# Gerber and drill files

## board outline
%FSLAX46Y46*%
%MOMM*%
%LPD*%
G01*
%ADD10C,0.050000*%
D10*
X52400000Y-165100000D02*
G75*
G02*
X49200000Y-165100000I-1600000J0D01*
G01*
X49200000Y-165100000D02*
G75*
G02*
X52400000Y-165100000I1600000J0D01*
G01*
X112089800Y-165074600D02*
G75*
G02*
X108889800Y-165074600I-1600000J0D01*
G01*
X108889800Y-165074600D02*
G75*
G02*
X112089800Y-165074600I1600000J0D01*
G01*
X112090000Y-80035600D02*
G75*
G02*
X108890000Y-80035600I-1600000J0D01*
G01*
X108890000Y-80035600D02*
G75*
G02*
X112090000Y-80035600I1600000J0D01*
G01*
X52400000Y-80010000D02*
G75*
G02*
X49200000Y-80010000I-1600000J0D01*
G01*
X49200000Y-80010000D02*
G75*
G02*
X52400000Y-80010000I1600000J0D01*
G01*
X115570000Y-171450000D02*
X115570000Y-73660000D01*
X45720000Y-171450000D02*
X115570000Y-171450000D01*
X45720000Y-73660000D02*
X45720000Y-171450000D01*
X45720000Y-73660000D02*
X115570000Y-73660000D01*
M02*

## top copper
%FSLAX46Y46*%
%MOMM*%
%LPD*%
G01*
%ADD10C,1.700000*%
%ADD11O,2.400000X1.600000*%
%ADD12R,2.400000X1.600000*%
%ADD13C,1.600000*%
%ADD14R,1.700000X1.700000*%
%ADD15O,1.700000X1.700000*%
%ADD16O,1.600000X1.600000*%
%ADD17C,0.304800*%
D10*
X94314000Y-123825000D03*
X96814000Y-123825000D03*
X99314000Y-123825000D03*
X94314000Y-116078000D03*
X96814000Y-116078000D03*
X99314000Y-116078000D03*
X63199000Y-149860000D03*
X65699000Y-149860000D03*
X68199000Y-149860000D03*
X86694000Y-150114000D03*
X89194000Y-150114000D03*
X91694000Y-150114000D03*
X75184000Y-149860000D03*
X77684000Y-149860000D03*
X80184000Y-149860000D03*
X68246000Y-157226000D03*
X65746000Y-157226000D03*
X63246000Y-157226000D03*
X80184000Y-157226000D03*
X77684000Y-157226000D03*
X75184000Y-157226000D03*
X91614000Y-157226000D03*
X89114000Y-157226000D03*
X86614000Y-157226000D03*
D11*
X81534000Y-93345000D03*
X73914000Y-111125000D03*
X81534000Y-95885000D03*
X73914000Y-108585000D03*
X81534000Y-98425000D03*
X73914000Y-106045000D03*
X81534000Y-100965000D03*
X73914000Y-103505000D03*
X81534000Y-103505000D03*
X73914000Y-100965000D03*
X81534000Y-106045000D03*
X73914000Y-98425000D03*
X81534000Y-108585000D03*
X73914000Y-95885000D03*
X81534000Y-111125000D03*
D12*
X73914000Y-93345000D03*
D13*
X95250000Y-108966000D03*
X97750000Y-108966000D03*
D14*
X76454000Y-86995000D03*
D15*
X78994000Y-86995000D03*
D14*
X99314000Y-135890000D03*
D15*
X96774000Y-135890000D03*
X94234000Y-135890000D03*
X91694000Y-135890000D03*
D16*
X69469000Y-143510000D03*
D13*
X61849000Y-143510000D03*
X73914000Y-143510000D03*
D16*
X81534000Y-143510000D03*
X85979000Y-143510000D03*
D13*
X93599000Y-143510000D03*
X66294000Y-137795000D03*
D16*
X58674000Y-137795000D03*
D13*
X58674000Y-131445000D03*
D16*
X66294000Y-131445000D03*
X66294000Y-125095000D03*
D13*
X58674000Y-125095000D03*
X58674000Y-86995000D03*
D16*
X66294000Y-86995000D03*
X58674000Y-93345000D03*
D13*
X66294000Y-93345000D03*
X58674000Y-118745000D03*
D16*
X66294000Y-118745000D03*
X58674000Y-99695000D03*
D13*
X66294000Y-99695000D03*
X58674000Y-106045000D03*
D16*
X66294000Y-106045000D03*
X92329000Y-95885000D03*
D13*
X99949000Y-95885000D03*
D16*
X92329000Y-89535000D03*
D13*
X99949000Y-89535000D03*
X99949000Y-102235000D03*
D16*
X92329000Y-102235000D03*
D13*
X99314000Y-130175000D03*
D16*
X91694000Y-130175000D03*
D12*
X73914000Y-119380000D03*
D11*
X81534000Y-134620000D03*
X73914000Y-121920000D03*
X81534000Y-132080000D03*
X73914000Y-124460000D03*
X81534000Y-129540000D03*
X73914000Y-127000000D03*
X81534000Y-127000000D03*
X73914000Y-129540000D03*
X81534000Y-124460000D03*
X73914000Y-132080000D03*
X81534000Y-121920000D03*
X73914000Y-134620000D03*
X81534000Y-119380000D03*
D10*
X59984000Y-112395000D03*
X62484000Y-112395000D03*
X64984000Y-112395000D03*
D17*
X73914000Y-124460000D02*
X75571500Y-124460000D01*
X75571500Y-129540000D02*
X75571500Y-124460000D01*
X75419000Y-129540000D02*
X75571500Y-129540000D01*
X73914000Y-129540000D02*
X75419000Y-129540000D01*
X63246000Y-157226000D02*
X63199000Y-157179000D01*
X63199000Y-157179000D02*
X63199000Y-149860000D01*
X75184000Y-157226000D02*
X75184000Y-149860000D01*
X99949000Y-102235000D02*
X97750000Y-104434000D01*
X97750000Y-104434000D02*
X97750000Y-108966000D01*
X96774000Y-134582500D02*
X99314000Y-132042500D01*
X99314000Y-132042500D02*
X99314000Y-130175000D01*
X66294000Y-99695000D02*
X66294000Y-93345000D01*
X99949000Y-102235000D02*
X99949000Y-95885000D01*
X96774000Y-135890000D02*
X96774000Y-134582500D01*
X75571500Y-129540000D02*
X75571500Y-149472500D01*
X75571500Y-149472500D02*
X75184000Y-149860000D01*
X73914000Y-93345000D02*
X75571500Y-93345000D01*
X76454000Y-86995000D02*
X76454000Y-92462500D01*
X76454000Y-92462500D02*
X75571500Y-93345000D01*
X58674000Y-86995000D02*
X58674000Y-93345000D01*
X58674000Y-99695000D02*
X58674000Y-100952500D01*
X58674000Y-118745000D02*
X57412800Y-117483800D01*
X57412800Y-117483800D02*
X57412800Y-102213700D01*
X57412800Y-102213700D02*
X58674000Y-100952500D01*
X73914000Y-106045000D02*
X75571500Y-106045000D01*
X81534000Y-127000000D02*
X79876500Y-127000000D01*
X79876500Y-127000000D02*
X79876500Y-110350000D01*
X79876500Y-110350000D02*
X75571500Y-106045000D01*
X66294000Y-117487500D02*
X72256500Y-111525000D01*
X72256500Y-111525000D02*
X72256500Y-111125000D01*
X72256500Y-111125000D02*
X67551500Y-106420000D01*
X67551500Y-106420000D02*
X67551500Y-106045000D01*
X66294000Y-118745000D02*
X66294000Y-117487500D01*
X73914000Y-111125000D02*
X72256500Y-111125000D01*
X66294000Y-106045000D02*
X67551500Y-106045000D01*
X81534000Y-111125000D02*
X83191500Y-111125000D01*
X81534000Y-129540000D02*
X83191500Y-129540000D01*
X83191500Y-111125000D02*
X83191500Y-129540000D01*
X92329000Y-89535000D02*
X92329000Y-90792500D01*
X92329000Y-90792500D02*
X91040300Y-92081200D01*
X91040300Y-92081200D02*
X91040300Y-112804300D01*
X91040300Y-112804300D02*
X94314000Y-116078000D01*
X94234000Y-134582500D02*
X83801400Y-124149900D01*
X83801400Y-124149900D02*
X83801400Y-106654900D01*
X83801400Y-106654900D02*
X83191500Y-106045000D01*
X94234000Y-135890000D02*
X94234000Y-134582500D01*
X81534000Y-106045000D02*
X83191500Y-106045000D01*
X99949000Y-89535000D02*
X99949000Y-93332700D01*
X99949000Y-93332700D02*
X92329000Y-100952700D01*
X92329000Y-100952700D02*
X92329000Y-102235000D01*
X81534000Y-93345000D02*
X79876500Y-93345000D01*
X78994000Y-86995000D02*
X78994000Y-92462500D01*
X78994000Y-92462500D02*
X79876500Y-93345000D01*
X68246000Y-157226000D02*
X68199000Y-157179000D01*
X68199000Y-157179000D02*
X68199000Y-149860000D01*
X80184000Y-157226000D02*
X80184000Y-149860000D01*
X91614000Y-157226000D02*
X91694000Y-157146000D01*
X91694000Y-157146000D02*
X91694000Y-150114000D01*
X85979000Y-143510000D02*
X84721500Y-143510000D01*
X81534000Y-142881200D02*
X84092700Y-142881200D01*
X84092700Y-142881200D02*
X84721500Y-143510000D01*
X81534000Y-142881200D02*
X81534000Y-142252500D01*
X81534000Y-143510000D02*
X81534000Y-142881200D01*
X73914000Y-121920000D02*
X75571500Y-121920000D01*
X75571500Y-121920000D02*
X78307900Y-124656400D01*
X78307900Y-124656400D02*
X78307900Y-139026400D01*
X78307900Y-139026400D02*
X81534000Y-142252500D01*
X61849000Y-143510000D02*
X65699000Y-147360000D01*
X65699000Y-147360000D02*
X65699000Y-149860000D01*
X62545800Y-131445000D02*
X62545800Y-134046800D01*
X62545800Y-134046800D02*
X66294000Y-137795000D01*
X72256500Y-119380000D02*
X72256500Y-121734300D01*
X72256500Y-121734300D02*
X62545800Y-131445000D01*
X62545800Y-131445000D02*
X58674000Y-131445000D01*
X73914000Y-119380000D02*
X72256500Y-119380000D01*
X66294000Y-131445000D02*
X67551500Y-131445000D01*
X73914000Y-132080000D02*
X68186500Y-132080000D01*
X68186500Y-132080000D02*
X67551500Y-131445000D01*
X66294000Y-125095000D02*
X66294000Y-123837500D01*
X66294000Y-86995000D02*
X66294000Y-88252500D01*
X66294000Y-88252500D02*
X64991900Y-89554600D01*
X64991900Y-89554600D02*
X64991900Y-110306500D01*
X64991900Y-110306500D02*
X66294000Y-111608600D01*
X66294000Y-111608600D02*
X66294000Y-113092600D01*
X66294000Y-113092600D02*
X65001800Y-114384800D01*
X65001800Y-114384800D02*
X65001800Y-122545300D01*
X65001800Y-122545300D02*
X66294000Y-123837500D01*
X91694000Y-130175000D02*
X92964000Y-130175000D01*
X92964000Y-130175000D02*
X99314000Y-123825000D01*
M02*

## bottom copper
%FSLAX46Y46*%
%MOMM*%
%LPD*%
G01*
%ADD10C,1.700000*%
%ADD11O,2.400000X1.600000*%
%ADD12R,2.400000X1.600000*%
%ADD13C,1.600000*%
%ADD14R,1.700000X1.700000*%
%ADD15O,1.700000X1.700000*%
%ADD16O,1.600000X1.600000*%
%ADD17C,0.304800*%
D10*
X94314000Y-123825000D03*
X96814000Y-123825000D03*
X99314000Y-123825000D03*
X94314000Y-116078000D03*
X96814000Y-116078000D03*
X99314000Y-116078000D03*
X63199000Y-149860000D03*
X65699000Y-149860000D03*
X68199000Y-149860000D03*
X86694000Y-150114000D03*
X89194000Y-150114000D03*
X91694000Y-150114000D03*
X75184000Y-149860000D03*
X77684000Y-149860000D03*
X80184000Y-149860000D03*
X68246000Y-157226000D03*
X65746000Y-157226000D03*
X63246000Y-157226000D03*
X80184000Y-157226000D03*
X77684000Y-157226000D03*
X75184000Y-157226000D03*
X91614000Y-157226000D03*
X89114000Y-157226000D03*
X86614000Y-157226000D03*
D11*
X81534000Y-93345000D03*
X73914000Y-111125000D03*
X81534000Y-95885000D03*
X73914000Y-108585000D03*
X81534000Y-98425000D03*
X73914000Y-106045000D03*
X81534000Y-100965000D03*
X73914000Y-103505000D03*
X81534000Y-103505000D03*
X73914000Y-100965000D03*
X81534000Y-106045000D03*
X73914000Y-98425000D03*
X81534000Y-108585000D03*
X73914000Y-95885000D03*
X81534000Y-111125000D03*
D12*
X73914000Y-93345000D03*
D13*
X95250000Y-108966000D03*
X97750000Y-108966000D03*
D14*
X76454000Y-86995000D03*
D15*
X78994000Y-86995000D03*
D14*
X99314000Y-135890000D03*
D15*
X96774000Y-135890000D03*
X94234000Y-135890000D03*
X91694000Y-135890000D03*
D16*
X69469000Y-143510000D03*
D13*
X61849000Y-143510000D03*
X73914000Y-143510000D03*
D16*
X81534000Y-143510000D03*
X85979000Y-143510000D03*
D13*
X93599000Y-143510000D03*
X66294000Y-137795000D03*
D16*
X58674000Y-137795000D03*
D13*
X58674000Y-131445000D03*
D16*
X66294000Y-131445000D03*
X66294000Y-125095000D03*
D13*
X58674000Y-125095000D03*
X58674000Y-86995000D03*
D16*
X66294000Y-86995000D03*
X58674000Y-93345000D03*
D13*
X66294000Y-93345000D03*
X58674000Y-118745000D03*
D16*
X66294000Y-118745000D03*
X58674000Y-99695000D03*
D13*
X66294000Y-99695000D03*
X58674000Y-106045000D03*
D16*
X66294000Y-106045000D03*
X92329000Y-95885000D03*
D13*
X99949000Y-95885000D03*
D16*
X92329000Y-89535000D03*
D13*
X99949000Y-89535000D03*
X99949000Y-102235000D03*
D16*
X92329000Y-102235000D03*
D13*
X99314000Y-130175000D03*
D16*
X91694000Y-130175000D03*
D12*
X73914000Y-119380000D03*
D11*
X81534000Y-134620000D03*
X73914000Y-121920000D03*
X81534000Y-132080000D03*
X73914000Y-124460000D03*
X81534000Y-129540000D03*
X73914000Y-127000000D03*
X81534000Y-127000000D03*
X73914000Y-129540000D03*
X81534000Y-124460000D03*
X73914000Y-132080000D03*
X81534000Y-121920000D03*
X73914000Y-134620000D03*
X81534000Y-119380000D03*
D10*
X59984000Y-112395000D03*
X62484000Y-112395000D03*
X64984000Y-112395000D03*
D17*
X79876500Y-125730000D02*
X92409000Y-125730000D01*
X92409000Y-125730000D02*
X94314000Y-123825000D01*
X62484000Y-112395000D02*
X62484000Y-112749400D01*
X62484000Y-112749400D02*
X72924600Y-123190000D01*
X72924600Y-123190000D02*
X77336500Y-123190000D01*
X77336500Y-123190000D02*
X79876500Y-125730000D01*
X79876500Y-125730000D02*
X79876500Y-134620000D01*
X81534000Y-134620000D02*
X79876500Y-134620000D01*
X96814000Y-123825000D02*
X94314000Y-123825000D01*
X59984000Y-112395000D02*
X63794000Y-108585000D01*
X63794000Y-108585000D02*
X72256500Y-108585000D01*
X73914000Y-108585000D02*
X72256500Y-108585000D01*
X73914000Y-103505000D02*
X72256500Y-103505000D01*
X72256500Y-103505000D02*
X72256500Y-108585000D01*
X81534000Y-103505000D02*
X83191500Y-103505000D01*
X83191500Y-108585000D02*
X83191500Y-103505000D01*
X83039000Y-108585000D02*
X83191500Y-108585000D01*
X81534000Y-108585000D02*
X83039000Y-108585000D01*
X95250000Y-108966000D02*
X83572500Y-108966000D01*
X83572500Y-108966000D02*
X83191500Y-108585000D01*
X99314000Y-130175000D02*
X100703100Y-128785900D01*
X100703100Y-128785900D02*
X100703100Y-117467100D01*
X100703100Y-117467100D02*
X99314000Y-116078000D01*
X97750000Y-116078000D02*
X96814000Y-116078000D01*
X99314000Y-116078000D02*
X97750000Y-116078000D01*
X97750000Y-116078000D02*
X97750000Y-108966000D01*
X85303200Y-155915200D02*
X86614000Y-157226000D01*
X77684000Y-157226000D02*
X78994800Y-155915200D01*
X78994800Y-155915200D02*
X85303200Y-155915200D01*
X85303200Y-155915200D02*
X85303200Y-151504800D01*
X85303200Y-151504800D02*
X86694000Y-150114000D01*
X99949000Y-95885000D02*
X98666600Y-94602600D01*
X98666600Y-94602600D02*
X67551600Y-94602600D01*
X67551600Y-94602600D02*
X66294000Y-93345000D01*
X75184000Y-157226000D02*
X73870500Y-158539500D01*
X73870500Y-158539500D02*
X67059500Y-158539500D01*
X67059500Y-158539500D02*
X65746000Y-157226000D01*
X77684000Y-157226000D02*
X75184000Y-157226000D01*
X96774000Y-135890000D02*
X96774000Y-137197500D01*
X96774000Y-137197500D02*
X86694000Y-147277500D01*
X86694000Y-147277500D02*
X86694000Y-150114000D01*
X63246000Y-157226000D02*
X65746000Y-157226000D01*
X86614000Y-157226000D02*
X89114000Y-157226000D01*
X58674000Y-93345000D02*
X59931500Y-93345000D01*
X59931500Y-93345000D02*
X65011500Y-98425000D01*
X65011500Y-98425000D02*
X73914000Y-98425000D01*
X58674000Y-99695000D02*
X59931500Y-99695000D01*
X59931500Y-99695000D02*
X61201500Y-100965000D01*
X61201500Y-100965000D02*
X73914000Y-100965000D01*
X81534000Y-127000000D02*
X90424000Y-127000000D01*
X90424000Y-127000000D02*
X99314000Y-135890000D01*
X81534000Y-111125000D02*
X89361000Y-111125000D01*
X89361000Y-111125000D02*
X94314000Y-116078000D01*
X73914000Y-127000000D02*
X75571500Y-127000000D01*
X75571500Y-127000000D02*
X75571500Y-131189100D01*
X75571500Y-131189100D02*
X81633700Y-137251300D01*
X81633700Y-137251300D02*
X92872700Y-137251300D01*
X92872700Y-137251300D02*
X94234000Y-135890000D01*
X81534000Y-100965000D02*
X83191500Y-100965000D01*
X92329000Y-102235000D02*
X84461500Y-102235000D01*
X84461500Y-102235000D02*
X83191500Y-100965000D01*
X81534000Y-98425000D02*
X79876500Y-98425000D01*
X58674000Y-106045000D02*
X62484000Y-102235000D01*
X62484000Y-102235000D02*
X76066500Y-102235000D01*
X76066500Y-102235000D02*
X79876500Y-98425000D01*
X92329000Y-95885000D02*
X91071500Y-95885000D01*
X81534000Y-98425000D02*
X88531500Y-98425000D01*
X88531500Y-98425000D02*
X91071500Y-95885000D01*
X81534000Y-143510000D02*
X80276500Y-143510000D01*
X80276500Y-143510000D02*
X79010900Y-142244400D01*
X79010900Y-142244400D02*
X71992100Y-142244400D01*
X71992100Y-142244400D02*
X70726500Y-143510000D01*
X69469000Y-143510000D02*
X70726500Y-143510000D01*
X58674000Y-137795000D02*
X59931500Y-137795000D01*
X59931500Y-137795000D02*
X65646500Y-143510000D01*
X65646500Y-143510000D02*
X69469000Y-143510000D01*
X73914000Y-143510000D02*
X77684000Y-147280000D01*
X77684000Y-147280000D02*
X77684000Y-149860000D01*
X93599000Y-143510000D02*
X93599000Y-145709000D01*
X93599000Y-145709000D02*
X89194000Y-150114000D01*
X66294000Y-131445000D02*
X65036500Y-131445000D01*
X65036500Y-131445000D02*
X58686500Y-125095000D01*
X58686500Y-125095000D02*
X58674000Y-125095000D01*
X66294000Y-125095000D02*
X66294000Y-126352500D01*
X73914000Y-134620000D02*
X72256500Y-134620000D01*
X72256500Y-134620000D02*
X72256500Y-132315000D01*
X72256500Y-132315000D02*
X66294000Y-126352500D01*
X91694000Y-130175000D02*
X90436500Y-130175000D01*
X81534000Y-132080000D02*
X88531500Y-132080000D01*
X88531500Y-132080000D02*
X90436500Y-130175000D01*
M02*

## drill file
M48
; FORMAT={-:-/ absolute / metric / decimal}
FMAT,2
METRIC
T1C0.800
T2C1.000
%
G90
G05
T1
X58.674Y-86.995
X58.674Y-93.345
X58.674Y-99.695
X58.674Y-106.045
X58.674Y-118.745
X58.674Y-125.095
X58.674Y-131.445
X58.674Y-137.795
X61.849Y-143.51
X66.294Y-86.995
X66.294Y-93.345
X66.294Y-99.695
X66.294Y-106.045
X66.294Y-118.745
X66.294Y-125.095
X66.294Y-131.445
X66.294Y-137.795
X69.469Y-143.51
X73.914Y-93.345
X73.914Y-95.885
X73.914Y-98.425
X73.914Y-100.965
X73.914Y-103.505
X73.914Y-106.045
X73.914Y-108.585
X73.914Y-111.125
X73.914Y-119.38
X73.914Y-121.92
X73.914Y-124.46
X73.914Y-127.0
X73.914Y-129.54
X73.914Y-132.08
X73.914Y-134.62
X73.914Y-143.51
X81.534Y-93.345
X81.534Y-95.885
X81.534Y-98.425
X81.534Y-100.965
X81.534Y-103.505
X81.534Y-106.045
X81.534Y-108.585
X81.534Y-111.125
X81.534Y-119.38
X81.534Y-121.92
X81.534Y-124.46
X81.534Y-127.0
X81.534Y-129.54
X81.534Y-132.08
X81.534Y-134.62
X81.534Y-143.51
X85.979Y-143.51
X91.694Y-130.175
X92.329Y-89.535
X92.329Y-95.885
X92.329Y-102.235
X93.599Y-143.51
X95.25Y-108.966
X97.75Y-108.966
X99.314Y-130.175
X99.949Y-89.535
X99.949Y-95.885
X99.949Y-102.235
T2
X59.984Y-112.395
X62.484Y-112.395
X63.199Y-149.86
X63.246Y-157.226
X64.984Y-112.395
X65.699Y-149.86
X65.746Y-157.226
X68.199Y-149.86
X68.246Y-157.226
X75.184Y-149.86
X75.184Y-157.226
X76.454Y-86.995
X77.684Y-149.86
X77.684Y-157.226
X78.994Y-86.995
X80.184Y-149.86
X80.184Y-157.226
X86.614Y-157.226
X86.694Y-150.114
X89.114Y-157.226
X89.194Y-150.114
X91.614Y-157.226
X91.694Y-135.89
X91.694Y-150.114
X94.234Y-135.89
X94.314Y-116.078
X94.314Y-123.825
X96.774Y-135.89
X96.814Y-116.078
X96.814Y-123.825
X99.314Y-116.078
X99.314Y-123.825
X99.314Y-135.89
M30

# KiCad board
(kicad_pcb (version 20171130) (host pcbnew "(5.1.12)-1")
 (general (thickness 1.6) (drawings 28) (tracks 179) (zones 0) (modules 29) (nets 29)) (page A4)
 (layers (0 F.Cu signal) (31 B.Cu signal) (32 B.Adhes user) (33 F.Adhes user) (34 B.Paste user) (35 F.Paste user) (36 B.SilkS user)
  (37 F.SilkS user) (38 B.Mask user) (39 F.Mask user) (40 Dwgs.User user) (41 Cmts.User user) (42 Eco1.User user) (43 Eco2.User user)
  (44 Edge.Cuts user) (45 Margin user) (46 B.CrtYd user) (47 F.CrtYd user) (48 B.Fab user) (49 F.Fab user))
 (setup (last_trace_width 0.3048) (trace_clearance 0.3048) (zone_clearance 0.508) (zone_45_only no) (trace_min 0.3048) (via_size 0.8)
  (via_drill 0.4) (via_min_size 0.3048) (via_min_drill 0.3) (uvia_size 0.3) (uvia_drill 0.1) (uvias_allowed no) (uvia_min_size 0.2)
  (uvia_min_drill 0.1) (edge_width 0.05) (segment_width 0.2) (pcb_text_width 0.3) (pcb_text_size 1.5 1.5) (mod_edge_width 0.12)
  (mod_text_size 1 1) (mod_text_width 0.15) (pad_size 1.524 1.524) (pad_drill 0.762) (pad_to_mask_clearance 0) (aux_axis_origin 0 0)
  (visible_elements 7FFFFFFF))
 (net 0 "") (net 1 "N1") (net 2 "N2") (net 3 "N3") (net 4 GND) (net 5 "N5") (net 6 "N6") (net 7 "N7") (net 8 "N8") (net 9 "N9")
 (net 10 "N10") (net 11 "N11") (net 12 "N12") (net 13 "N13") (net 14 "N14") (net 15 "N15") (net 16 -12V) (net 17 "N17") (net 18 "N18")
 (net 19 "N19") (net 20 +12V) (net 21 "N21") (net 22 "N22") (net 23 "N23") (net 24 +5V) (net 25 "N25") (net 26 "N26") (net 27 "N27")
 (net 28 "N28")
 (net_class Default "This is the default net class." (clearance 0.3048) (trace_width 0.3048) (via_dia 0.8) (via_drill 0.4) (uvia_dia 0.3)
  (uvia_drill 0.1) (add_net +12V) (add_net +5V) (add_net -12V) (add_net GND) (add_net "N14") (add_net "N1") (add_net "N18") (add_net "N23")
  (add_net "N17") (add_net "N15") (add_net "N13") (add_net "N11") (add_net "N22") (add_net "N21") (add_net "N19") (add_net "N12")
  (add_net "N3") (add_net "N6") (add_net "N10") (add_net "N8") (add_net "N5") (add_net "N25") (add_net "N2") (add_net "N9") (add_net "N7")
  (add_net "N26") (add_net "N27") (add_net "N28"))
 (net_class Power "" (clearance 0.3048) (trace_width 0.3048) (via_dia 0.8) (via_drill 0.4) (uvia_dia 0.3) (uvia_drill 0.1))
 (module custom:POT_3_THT (layer F.Cu) (at 99.314 123.825 180)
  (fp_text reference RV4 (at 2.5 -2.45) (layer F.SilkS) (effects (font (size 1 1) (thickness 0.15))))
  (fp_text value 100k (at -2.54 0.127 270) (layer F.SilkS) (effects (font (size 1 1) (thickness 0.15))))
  (pad 3 thru_hole circle (at 5 0 180) (size 1.7 1.7) (drill 1) (layers *.Cu *.Mask) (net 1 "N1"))
  (pad 2 thru_hole circle (at 2.5 0 180) (size 1.7 1.7) (drill 1) (layers *.Cu *.Mask) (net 1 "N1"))
  (pad 1 thru_hole circle (at 0 0 180) (size 1.7 1.7) (drill 1) (layers *.Cu *.Mask) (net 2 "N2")))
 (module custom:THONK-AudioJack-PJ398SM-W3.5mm (layer F.Cu) (at 99.314 116.078 180)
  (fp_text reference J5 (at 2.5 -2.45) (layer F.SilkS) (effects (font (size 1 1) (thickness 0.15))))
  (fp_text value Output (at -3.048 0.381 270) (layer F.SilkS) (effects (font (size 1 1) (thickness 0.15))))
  (pad TN thru_hole circle (at 5 0 180) (size 1.7 1.7) (drill 1) (layers *.Cu *.Mask) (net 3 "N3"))
  (pad T thru_hole circle (at 2.5 0 180) (size 1.7 1.7) (drill 1) (layers *.Cu *.Mask) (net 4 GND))
  (pad S thru_hole circle (at 0 0 180) (size 1.7 1.7) (drill 1) (layers *.Cu *.Mask) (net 4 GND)))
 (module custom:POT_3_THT (layer F.Cu) (at 68.199 149.86 180)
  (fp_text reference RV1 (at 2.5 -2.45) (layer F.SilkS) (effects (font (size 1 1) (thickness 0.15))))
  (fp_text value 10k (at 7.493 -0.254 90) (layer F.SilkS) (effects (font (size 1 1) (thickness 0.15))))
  (pad 3 thru_hole circle (at 5 0 180) (size 1.7 1.7) (drill 1) (layers *.Cu *.Mask) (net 4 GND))
  (pad 2 thru_hole circle (at 2.5 0 180) (size 1.7 1.7) (drill 1) (layers *.Cu *.Mask) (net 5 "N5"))
  (pad 1 thru_hole circle (at 0 0 180) (size 1.7 1.7) (drill 1) (layers *.Cu *.Mask) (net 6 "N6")))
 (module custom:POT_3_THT (layer F.Cu) (at 91.694 150.114 180)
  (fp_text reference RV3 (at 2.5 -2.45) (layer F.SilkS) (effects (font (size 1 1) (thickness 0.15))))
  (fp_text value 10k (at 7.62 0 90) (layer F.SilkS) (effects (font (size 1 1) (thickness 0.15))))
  (pad 3 thru_hole circle (at 5 0 180) (size 1.7 1.7) (drill 1) (layers *.Cu *.Mask) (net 4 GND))
  (pad 2 thru_hole circle (at 2.5 0 180) (size 1.7 1.7) (drill 1) (layers *.Cu *.Mask) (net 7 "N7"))
  (pad 1 thru_hole circle (at 0 0 180) (size 1.7 1.7) (drill 1) (layers *.Cu *.Mask) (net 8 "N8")))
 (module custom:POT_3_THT (layer F.Cu) (at 80.184 149.86 180)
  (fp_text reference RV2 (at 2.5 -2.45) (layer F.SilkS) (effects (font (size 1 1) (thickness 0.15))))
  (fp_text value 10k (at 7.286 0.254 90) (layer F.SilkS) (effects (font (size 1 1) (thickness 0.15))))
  (pad 3 thru_hole circle (at 5 0 180) (size 1.7 1.7) (drill 1) (layers *.Cu *.Mask) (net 4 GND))
  (pad 2 thru_hole circle (at 2.5 0 180) (size 1.7 1.7) (drill 1) (layers *.Cu *.Mask) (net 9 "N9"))
  (pad 1 thru_hole circle (at 0 0 180) (size 1.7 1.7) (drill 1) (layers *.Cu *.Mask) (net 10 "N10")))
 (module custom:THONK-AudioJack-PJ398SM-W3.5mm (layer F.Cu) (at 63.246 157.226)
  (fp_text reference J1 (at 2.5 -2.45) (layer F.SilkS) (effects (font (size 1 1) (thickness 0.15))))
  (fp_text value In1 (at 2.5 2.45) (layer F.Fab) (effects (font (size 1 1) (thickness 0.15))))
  (pad TN thru_hole circle (at 5 0) (size 1.7 1.7) (drill 1) (layers *.Cu *.Mask) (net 6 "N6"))
  (pad T thru_hole circle (at 2.5 0) (size 1.7 1.7) (drill 1) (layers *.Cu *.Mask) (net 4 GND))
  (pad S thru_hole circle (at 0 0) (size 1.7 1.7) (drill 1) (layers *.Cu *.Mask) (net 4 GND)))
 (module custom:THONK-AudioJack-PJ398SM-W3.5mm (layer F.Cu) (at 75.184 157.226)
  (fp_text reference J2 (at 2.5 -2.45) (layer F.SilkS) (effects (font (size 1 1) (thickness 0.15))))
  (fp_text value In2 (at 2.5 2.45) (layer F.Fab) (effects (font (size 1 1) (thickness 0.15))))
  (pad TN thru_hole circle (at 5 0) (size 1.7 1.7) (drill 1) (layers *.Cu *.Mask) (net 10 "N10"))
  (pad T thru_hole circle (at 2.5 0) (size 1.7 1.7) (drill 1) (layers *.Cu *.Mask) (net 4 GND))
  (pad S thru_hole circle (at 0 0) (size 1.7 1.7) (drill 1) (layers *.Cu *.Mask) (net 4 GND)))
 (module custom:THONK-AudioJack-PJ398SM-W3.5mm (layer F.Cu) (at 86.614 157.226)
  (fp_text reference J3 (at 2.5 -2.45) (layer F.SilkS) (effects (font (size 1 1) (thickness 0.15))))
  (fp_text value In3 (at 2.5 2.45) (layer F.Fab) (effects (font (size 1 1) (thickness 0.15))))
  (pad TN thru_hole circle (at 5 0) (size 1.7 1.7) (drill 1) (layers *.Cu *.Mask) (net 8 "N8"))
  (pad T thru_hole circle (at 2.5 0) (size 1.7 1.7) (drill 1) (layers *.Cu *.Mask) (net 4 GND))
  (pad S thru_hole circle (at 0 0) (size 1.7 1.7) (drill 1) (layers *.Cu *.Mask) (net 4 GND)))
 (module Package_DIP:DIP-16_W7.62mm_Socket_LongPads (layer F.Cu) (at 73.914 93.345)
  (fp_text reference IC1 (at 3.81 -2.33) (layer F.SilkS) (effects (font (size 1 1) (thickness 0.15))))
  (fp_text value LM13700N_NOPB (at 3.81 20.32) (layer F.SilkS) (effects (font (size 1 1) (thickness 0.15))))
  (pad 16 thru_hole oval (at 7.62 0) (size 2.4 1.6) (drill 0.8) (layers *.Cu *.Mask) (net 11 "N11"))
  (pad 8 thru_hole oval (at 0 17.78) (size 2.4 1.6) (drill 0.8) (layers *.Cu *.Mask) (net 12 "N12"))
  (pad 15 thru_hole oval (at 7.62 2.54) (size 2.4 1.6) (drill 0.8) (layers *.Cu *.Mask) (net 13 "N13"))
  (pad 7 thru_hole oval (at 0 15.24) (size 2.4 1.6) (drill 0.8) (layers *.Cu *.Mask) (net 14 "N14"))
  (pad 14 thru_hole oval (at 7.62 5.08) (size 2.4 1.6) (drill 0.8) (layers *.Cu *.Mask) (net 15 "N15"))
  (pad 6 thru_hole oval (at 0 12.7) (size 2.4 1.6) (drill 0.8) (layers *.Cu *.Mask) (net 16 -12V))
  (pad 13 thru_hole oval (at 7.62 7.62) (size 2.4 1.6) (drill 0.8) (layers *.Cu *.Mask) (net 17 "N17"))
  (pad 5 thru_hole oval (at 0 10.16) (size 2.4 1.6) (drill 0.8) (layers *.Cu *.Mask) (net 14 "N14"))
  (pad 12 thru_hole oval (at 7.62 10.16) (size 2.4 1.6) (drill 0.8) (layers *.Cu *.Mask) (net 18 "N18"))
  (pad 4 thru_hole oval (at 0 7.62) (size 2.4 1.6) (drill 0.8) (layers *.Cu *.Mask) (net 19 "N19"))
  (pad 11 thru_hole oval (at 7.62 12.7) (size 2.4 1.6) (drill 0.8) (layers *.Cu *.Mask) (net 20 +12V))
  (pad 3 thru_hole oval (at 0 5.08) (size 2.4 1.6) (drill 0.8) (layers *.Cu *.Mask) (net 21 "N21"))
  (pad 10 thru_hole oval (at 7.62 15.24) (size 2.4 1.6) (drill 0.8) (layers *.Cu *.Mask) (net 18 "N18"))
  (pad 2 thru_hole oval (at 0 2.54) (size 2.4 1.6) (drill 0.8) (layers *.Cu *.Mask) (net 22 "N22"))
  (pad 9 thru_hole oval (at 7.62 17.78) (size 2.4 1.6) (drill 0.8) (layers *.Cu *.Mask) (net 3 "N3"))
  (pad 1 thru_hole rect (at 0 0) (size 2.4 1.6) (drill 0.8) (layers *.Cu *.Mask) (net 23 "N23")))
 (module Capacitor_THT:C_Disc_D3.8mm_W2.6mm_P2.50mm (layer F.Cu) (at 95.25 108.966)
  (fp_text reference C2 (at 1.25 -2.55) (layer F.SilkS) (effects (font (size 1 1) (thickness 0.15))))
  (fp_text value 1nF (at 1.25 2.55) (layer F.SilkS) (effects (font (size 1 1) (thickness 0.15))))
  (pad 1 thru_hole circle (at 0 0) (size 1.6 1.6) (drill 0.8) (layers *.Cu *.Mask) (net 18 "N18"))
  (pad 2 thru_hole circle (at 2.5 0) (size 1.6 1.6) (drill 0.8) (layers *.Cu *.Mask) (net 4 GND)))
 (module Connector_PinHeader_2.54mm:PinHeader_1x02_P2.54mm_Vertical (layer F.Cu) (at 76.454 86.995 90)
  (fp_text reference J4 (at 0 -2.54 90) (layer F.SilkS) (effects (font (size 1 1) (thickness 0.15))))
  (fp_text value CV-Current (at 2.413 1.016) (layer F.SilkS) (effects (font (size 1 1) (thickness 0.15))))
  (pad 1 thru_hole rect (at 0 0 90) (size 1.7 1.7) (drill 1) (layers *.Cu *.Mask) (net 23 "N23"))
  (pad 2 thru_hole oval (at 0 2.54 90) (size 1.7 1.7) (drill 1) (layers *.Cu *.Mask) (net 11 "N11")))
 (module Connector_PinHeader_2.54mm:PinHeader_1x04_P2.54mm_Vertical (layer F.Cu) (at 99.314 135.89 270)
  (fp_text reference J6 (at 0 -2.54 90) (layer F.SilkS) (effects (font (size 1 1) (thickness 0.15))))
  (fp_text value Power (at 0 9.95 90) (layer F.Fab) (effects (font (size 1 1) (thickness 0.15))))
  (pad 1 thru_hole rect (at 0 0 270) (size 1.7 1.7) (drill 1) (layers *.Cu *.Mask) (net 16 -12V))
  (pad 2 thru_hole oval (at 0 2.54 270) (size 1.7 1.7) (drill 1) (layers *.Cu *.Mask) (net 4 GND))
  (pad 3 thru_hole oval (at 0 5.08 270) (size 1.7 1.7) (drill 1) (layers *.Cu *.Mask) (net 20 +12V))
  (pad 4 thru_hole oval (at 0 7.62 270) (size 1.7 1.7) (drill 1) (layers *.Cu *.Mask) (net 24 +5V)))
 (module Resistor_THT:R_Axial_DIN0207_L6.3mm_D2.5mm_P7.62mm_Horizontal (layer F.Cu) (at 61.849 143.51)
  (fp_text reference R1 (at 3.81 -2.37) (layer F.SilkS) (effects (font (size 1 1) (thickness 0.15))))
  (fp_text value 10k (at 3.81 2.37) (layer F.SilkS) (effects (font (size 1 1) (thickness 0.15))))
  (pad 2 thru_hole oval (at 7.62 0) (size 1.6 1.6) (drill 0.8) (layers *.Cu *.Mask) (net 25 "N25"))
  (pad 1 thru_hole circle (at 0 0) (size 1.6 1.6) (drill 0.8) (layers *.Cu *.Mask) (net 5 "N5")))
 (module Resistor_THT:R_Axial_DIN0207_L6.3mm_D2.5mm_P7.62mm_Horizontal (layer F.Cu) (at 73.914 143.51)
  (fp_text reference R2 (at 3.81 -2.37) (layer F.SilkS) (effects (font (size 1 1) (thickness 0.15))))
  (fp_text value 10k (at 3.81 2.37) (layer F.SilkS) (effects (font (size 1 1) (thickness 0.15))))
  (pad 1 thru_hole circle (at 0 0) (size 1.6 1.6) (drill 0.8) (layers *.Cu *.Mask) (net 9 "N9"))
  (pad 2 thru_hole oval (at 7.62 0) (size 1.6 1.6) (drill 0.8) (layers *.Cu *.Mask) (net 25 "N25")))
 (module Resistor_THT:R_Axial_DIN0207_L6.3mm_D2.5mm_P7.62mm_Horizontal (layer F.Cu) (at 93.599 143.51 180)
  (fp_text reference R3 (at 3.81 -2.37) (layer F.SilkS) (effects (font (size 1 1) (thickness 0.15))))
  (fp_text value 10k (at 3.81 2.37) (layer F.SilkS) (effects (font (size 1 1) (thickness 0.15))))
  (pad 2 thru_hole oval (at 7.62 0 180) (size 1.6 1.6) (drill 0.8) (layers *.Cu *.Mask) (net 25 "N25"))
  (pad 1 thru_hole circle (at 0 0 180) (size 1.6 1.6) (drill 0.8) (layers *.Cu *.Mask) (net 7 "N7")))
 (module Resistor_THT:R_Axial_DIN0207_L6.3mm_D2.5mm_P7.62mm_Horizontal (layer F.Cu) (at 66.294 137.795 180)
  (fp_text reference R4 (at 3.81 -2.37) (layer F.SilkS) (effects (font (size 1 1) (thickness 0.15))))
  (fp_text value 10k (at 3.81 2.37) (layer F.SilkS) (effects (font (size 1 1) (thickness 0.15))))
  (pad 1 thru_hole circle (at 0 0 180) (size 1.6 1.6) (drill 0.8) (layers *.Cu *.Mask) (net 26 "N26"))
  (pad 2 thru_hole oval (at 7.62 0 180) (size 1.6 1.6) (drill 0.8) (layers *.Cu *.Mask) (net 25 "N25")))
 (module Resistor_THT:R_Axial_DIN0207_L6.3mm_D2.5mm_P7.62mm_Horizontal (layer F.Cu) (at 58.674 131.445)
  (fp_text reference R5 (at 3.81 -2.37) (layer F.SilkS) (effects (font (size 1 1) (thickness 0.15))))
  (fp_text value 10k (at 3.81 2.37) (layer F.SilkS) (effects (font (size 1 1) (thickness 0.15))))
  (pad 1 thru_hole circle (at 0 0) (size 1.6 1.6) (drill 0.8) (layers *.Cu *.Mask) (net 26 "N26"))
  (pad 2 thru_hole oval (at 7.62 0) (size 1.6 1.6) (drill 0.8) (layers *.Cu *.Mask) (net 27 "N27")))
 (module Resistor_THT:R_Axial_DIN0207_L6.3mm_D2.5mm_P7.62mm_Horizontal (layer F.Cu) (at 58.674 125.095)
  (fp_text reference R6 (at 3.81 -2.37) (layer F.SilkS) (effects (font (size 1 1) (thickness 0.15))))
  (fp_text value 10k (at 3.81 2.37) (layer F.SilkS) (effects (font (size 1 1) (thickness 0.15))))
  (pad 2 thru_hole oval (at 7.62 0) (size 1.6 1.6) (drill 0.8) (layers *.Cu *.Mask) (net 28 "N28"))
  (pad 1 thru_hole circle (at 0 0) (size 1.6 1.6) (drill 0.8) (layers *.Cu *.Mask) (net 27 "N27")))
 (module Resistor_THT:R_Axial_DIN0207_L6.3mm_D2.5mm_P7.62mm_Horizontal (layer F.Cu) (at 58.674 86.995)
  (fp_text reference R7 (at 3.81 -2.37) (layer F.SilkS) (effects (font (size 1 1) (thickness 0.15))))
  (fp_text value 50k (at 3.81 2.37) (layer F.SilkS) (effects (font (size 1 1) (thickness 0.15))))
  (pad 1 thru_hole circle (at 0 0) (size 1.6 1.6) (drill 0.8) (layers *.Cu *.Mask) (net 21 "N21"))
  (pad 2 thru_hole oval (at 7.62 0) (size 1.6 1.6) (drill 0.8) (layers *.Cu *.Mask) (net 28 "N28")))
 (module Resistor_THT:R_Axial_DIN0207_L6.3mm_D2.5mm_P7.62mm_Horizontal (layer F.Cu) (at 66.294 93.345 180)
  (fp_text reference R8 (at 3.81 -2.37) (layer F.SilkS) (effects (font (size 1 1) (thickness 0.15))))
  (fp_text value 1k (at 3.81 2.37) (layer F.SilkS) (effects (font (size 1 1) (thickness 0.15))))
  (pad 2 thru_hole oval (at 7.62 0 180) (size 1.6 1.6) (drill 0.8) (layers *.Cu *.Mask) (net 21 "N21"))
  (pad 1 thru_hole circle (at 0 0 180) (size 1.6 1.6) (drill 0.8) (layers *.Cu *.Mask) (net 4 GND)))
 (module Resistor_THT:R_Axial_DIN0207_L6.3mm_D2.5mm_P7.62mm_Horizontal (layer F.Cu) (at 58.674 118.745)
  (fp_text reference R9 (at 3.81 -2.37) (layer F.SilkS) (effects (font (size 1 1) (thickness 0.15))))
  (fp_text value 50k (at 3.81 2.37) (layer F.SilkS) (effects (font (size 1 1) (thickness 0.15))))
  (pad 1 thru_hole circle (at 0 0) (size 1.6 1.6) (drill 0.8) (layers *.Cu *.Mask) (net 19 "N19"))
  (pad 2 thru_hole oval (at 7.62 0) (size 1.6 1.6) (drill 0.8) (layers *.Cu *.Mask) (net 12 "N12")))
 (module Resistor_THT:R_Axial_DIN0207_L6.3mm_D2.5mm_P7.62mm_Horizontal (layer F.Cu) (at 66.294 99.695 180)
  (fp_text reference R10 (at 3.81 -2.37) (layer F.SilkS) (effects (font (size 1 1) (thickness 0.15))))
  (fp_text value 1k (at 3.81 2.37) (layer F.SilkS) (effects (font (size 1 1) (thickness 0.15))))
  (pad 2 thru_hole oval (at 7.62 0 180) (size 1.6 1.6) (drill 0.8) (layers *.Cu *.Mask) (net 19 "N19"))
  (pad 1 thru_hole circle (at 0 0 180) (size 1.6 1.6) (drill 0.8) (layers *.Cu *.Mask) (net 4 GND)))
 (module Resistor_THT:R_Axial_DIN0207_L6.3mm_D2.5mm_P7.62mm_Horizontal (layer F.Cu) (at 58.674 106.045)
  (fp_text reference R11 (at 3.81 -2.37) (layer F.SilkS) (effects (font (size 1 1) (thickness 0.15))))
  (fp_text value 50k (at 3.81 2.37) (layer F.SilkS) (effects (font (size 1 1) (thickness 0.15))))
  (pad 1 thru_hole circle (at 0 0) (size 1.6 1.6) (drill 0.8) (layers *.Cu *.Mask) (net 15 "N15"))
  (pad 2 thru_hole oval (at 7.62 0) (size 1.6 1.6) (drill 0.8) (layers *.Cu *.Mask) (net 12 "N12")))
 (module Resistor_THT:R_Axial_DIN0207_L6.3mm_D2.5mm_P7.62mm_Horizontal (layer F.Cu) (at 99.949 95.885 180)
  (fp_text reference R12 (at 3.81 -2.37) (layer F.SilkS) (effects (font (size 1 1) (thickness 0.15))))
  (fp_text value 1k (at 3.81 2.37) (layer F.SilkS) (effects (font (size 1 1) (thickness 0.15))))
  (pad 2 thru_hole oval (at 7.62 0 180) (size 1.6 1.6) (drill 0.8) (layers *.Cu *.Mask) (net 15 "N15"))
  (pad 1 thru_hole circle (at 0 0 180) (size 1.6 1.6) (drill 0.8) (layers *.Cu *.Mask) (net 4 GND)))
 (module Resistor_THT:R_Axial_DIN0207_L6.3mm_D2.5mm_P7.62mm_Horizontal (layer F.Cu) (at 99.949 89.535 180)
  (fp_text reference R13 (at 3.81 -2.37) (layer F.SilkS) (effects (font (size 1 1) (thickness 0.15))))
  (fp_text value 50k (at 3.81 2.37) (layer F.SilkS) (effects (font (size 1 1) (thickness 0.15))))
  (pad 2 thru_hole oval (at 7.62 0 180) (size 1.6 1.6) (drill 0.8) (layers *.Cu *.Mask) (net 3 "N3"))
  (pad 1 thru_hole circle (at 0 0 180) (size 1.6 1.6) (drill 0.8) (layers *.Cu *.Mask) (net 17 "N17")))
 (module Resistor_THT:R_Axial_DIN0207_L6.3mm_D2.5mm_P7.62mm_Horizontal (layer F.Cu) (at 99.949 102.235 180)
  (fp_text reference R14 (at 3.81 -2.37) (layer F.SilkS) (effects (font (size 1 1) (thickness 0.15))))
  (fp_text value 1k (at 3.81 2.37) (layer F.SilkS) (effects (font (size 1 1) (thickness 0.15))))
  (pad 1 thru_hole circle (at 0 0 180) (size 1.6 1.6) (drill 0.8) (layers *.Cu *.Mask) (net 4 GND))
  (pad 2 thru_hole oval (at 7.62 0 180) (size 1.6 1.6) (drill 0.8) (layers *.Cu *.Mask) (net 17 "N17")))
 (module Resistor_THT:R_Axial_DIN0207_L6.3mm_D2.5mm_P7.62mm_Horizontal (layer F.Cu) (at 99.314 130.175 180)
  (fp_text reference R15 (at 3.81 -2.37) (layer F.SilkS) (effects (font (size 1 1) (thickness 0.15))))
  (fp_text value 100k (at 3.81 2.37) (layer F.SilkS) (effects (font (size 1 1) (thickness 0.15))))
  (pad 1 thru_hole circle (at 0 0 180) (size 1.6 1.6) (drill 0.8) (layers *.Cu *.Mask) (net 4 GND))
  (pad 2 thru_hole oval (at 7.62 0 180) (size 1.6 1.6) (drill 0.8) (layers *.Cu *.Mask) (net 2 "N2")))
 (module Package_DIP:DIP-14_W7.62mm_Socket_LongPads (layer F.Cu) (at 73.914 119.38)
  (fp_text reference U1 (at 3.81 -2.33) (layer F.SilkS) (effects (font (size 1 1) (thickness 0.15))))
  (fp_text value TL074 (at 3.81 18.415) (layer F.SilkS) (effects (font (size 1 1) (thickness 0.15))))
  (pad 1 thru_hole rect (at 0 0) (size 2.4 1.6) (drill 0.8) (layers *.Cu *.Mask) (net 26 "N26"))
  (pad 8 thru_hole oval (at 7.62 15.24) (size 2.4 1.6) (drill 0.8) (layers *.Cu *.Mask) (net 1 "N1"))
  (pad 2 thru_hole oval (at 0 2.54) (size 2.4 1.6) (drill 0.8) (layers *.Cu *.Mask) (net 25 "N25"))
  (pad 9 thru_hole oval (at 7.62 12.7) (size 2.4 1.6) (drill 0.8) (layers *.Cu *.Mask) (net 2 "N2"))
  (pad 3 thru_hole oval (at 0 5.08) (size 2.4 1.6) (drill 0.8) (layers *.Cu *.Mask) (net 4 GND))
  (pad 10 thru_hole oval (at 7.62 10.16) (size 2.4 1.6) (drill 0.8) (layers *.Cu *.Mask) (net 3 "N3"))
  (pad 4 thru_hole oval (at 0 7.62) (size 2.4 1.6) (drill 0.8) (layers *.Cu *.Mask) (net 20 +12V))
  (pad 11 thru_hole oval (at 7.62 7.62) (size 2.4 1.6) (drill 0.8) (layers *.Cu *.Mask) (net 16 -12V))
  (pad 5 thru_hole oval (at 0 10.16) (size 2.4 1.6) (drill 0.8) (layers *.Cu *.Mask) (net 4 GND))
  (pad 12 thru_hole oval (at 7.62 5.08) (size 2.4 1.6) (drill 0.8) (layers *.Cu *.Mask))
  (pad 6 thru_hole oval (at 0 12.7) (size 2.4 1.6) (drill 0.8) (layers *.Cu *.Mask) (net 27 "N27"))
  (pad 13 thru_hole oval (at 7.62 2.54) (size 2.4 1.6) (drill 0.8) (layers *.Cu *.Mask))
  (pad 7 thru_hole oval (at 0 15.24) (size 2.4 1.6) (drill 0.8) (layers *.Cu *.Mask) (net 28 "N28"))
  (pad 14 thru_hole oval (at 7.62 0) (size 2.4 1.6) (drill 0.8) (layers *.Cu *.Mask)))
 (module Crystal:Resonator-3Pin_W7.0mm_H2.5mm (layer F.Cu) (at 59.984 112.395)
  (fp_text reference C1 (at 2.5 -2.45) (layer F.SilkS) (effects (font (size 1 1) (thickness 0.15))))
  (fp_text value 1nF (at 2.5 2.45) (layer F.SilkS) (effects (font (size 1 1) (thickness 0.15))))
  (pad 1 thru_hole circle (at 0 0) (size 1.7 1.7) (drill 1) (layers *.Cu *.Mask) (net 14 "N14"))
  (pad 2 thru_hole circle (at 2.5 0) (size 1.7 1.7) (drill 1) (layers *.Cu *.Mask) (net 1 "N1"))
  (pad 3 thru_hole circle (at 5 0) (size 1.7 1.7) (drill 1) (layers *.Cu *.Mask)))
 (gr_circle (center 50.8 165.1) (end 52.4 165.1) (layer Edge.Cuts) (width 0.05))
 (gr_circle (center 110.4898 165.0746) (end 112.0898 165.0746) (layer Edge.Cuts) (width 0.05))
 (gr_circle (center 110.49 80.0356) (end 112.09 80.0356) (layer Edge.Cuts) (width 0.05))
 (gr_circle (center 50.8 80.01) (end 52.4 80.01) (layer Edge.Cuts) (width 0.05))
 (gr_line (start 115.57 171.45) (end 115.57 73.66) (layer Edge.Cuts) (width 0.05))
 (gr_line (start 45.72 171.45) (end 115.57 171.45) (layer Edge.Cuts) (width 0.05))
 (gr_line (start 45.72 73.66) (end 45.72 171.45) (layer Edge.Cuts) (width 0.05))
 (gr_line (start 45.72 73.66) (end 115.57 73.66) (layer Edge.Cuts) (width 0.05))
 (segment (start 79.8765 125.73) (end 92.409 125.73) (width 0.3048) (layer B.Cu) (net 1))
 (segment (start 92.409 125.73) (end 94.314 123.825) (width 0.3048) (layer B.Cu) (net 1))
 (segment (start 62.484 112.395) (end 62.484 112.7494) (width 0.3048) (layer B.Cu) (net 1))
 (segment (start 62.484 112.7494) (end 72.9246 123.19) (width 0.3048) (layer B.Cu) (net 1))
 (segment (start 72.9246 123.19) (end 77.3365 123.19) (width 0.3048) (layer B.Cu) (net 1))
 (segment (start 77.3365 123.19) (end 79.8765 125.73) (width 0.3048) (layer B.Cu) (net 1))
 (segment (start 79.8765 125.73) (end 79.8765 134.62) (width 0.3048) (layer B.Cu) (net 1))
 (segment (start 81.534 134.62) (end 79.8765 134.62) (width 0.3048) (layer B.Cu) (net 1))
 (segment (start 96.814 123.825) (end 94.314 123.825) (width 0.3048) (layer B.Cu) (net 1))
 (segment (start 59.984 112.395) (end 63.794 108.585) (width 0.3048) (layer B.Cu) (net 14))
 (segment (start 63.794 108.585) (end 72.2565 108.585) (width 0.3048) (layer B.Cu) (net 14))
 (segment (start 73.914 108.585) (end 72.2565 108.585) (width 0.3048) (layer B.Cu) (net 14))
 (segment (start 73.914 103.505) (end 72.2565 103.505) (width 0.3048) (layer B.Cu) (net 14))
 (segment (start 72.2565 103.505) (end 72.2565 108.585) (width 0.3048) (layer B.Cu) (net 14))
 (segment (start 81.534 103.505) (end 83.1915 103.505) (width 0.3048) (layer B.Cu) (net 18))
 (segment (start 83.1915 108.585) (end 83.1915 103.505) (width 0.3048) (layer B.Cu) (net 18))
 (segment (start 83.039 108.585) (end 83.1915 108.585) (width 0.3048) (layer B.Cu) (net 18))
 (segment (start 81.534 108.585) (end 83.039 108.585) (width 0.3048) (layer B.Cu) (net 18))
 (segment (start 95.25 108.966) (end 83.5725 108.966) (width 0.3048) (layer B.Cu) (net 18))
 (segment (start 83.5725 108.966) (end 83.1915 108.585) (width 0.3048) (layer B.Cu) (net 18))
 (segment (start 99.314 130.175) (end 100.7031 128.7859) (width 0.3048) (layer B.Cu) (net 4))
 (segment (start 100.7031 128.7859) (end 100.7031 117.4671) (width 0.3048) (layer B.Cu) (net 4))
 (segment (start 100.7031 117.4671) (end 99.314 116.078) (width 0.3048) (layer B.Cu) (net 4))
 (segment (start 97.75 116.078) (end 96.814 116.078) (width 0.3048) (layer B.Cu) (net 4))
 (segment (start 99.314 116.078) (end 97.75 116.078) (width 0.3048) (layer B.Cu) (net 4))
 (segment (start 97.75 116.078) (end 97.75 108.966) (width 0.3048) (layer B.Cu) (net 4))
 (segment (start 85.3032 155.9152) (end 86.614 157.226) (width 0.3048) (layer B.Cu) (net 4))
 (segment (start 77.684 157.226) (end 78.9948 155.9152) (width 0.3048) (layer B.Cu) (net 4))
 (segment (start 78.9948 155.9152) (end 85.3032 155.9152) (width 0.3048) (layer B.Cu) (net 4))
 (segment (start 85.3032 155.9152) (end 85.3032 151.5048) (width 0.3048) (layer B.Cu) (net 4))
 (segment (start 85.3032 151.5048) (end 86.694 150.114) (width 0.3048) (layer B.Cu) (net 4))
 (segment (start 73.914 124.46) (end 75.5715 124.46) (width 0.3048) (layer F.Cu) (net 4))
 (segment (start 75.5715 129.54) (end 75.5715 124.46) (width 0.3048) (layer F.Cu) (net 4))
 (segment (start 75.419 129.54) (end 75.5715 129.54) (width 0.3048) (layer F.Cu) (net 4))
 (segment (start 73.914 129.54) (end 75.419 129.54) (width 0.3048) (layer F.Cu) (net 4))
 (segment (start 99.949 95.885) (end 98.6666 94.6026) (width 0.3048) (layer B.Cu) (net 4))
 (segment (start 98.6666 94.6026) (end 67.5516 94.6026) (width 0.3048) (layer B.Cu) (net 4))
 (segment (start 67.5516 94.6026) (end 66.294 93.345) (width 0.3048) (layer B.Cu) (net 4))
 (segment (start 75.184 157.226) (end 73.8705 158.5395) (width 0.3048) (layer B.Cu) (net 4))
 (segment (start 73.8705 158.5395) (end 67.0595 158.5395) (width 0.3048) (layer B.Cu) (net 4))
 (segment (start 67.0595 158.5395) (end 65.746 157.226) (width 0.3048) (layer B.Cu) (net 4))
 (segment (start 77.684 157.226) (end 75.184 157.226) (width 0.3048) (layer B.Cu) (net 4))
 (segment (start 96.774 135.89) (end 96.774 137.1975) (width 0.3048) (layer B.Cu) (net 4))
 (segment (start 96.774 137.1975) (end 86.694 147.2775) (width 0.3048) (layer B.Cu) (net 4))
 (segment (start 86.694 147.2775) (end 86.694 150.114) (width 0.3048) (layer B.Cu) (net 4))
 (segment (start 63.246 157.226) (end 63.199 157.179) (width 0.3048) (layer F.Cu) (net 4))
 (segment (start 63.199 157.179) (end 63.199 149.86) (width 0.3048) (layer F.Cu) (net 4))
 (segment (start 63.246 157.226) (end 65.746 157.226) (width 0.3048) (layer B.Cu) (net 4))
 (segment (start 75.184 157.226) (end 75.184 149.86) (width 0.3048) (layer F.Cu) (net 4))
 (segment (start 86.614 157.226) (end 89.114 157.226) (width 0.3048) (layer B.Cu) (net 4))
 (segment (start 99.949 102.235) (end 97.75 104.434) (width 0.3048) (layer F.Cu) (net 4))
 (segment (start 97.75 104.434) (end 97.75 108.966) (width 0.3048) (layer F.Cu) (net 4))
 (segment (start 96.774 134.5825) (end 99.314 132.0425) (width 0.3048) (layer F.Cu) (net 4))
 (segment (start 99.314 132.0425) (end 99.314 130.175) (width 0.3048) (layer F.Cu) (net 4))
 (segment (start 66.294 99.695) (end 66.294 93.345) (width 0.3048) (layer F.Cu) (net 4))
 (segment (start 99.949 102.235) (end 99.949 95.885) (width 0.3048) (layer F.Cu) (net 4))
 (segment (start 96.774 135.89) (end 96.774 134.5825) (width 0.3048) (layer F.Cu) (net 4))
 (segment (start 75.5715 129.54) (end 75.5715 149.4725) (width 0.3048) (layer F.Cu) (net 4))
 (segment (start 75.5715 149.4725) (end 75.184 149.86) (width 0.3048) (layer F.Cu) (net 4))
 (segment (start 73.914 93.345) (end 75.5715 93.345) (width 0.3048) (layer F.Cu) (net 23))
 (segment (start 76.454 86.995) (end 76.454 92.4625) (width 0.3048) (layer F.Cu) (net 23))
 (segment (start 76.454 92.4625) (end 75.5715 93.345) (width 0.3048) (layer F.Cu) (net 23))
 (segment (start 58.674 93.345) (end 59.9315 93.345) (width 0.3048) (layer B.Cu) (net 21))
 (segment (start 59.9315 93.345) (end 65.0115 98.425) (width 0.3048) (layer B.Cu) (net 21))
 (segment (start 65.0115 98.425) (end 73.914 98.425) (width 0.3048) (layer B.Cu) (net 21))
 (segment (start 58.674 86.995) (end 58.674 93.345) (width 0.3048) (layer F.Cu) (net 21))
 (segment (start 58.674 99.695) (end 59.9315 99.695) (width 0.3048) (layer B.Cu) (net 19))
 (segment (start 59.9315 99.695) (end 61.2015 100.965) (width 0.3048) (layer B.Cu) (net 19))
 (segment (start 61.2015 100.965) (end 73.914 100.965) (width 0.3048) (layer B.Cu) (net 19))
 (segment (start 58.674 99.695) (end 58.674 100.9525) (width 0.3048) (layer F.Cu) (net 19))
 (segment (start 58.674 118.745) (end 57.4128 117.4838) (width 0.3048) (layer F.Cu) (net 19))
 (segment (start 57.4128 117.4838) (end 57.4128 102.2137) (width 0.3048) (layer F.Cu) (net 19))
 (segment (start 57.4128 102.2137) (end 58.674 100.9525) (width 0.3048) (layer F.Cu) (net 19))
 (segment (start 81.534 127) (end 90.424 127) (width 0.3048) (layer B.Cu) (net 16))
 (segment (start 90.424 127) (end 99.314 135.89) (width 0.3048) (layer B.Cu) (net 16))
 (segment (start 73.914 106.045) (end 75.5715 106.045) (width 0.3048) (layer F.Cu) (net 16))
 (segment (start 81.534 127) (end 79.8765 127) (width 0.3048) (layer F.Cu) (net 16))
 (segment (start 79.8765 127) (end 79.8765 110.35) (width 0.3048) (layer F.Cu) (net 16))
 (segment (start 79.8765 110.35) (end 75.5715 106.045) (width 0.3048) (layer F.Cu) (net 16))
 (segment (start 66.294 117.4875) (end 72.2565 111.525) (width 0.3048) (layer F.Cu) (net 12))
 (segment (start 72.2565 111.525) (end 72.2565 111.125) (width 0.3048) (layer F.Cu) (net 12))
 (segment (start 72.2565 111.125) (end 67.5515 106.42) (width 0.3048) (layer F.Cu) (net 12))
 (segment (start 67.5515 106.42) (end 67.5515 106.045) (width 0.3048) (layer F.Cu) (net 12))
 (segment (start 66.294 118.745) (end 66.294 117.4875) (width 0.3048) (layer F.Cu) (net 12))
 (segment (start 73.914 111.125) (end 72.2565 111.125) (width 0.3048) (layer F.Cu) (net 12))
 (segment (start 66.294 106.045) (end 67.5515 106.045) (width 0.3048) (layer F.Cu) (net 12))
 (segment (start 81.534 111.125) (end 83.1915 111.125) (width 0.3048) (layer F.Cu) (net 3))
 (segment (start 81.534 129.54) (end 83.1915 129.54) (width 0.3048) (layer F.Cu) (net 3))
 (segment (start 83.1915 111.125) (end 83.1915 129.54) (width 0.3048) (layer F.Cu) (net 3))
 (segment (start 81.534 111.125) (end 89.361 111.125) (width 0.3048) (layer B.Cu) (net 3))
 (segment (start 89.361 111.125) (end 94.314 116.078) (width 0.3048) (layer B.Cu) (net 3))
 (segment (start 92.329 89.535) (end 92.329 90.7925) (width 0.3048) (layer F.Cu) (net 3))
 (segment (start 92.329 90.7925) (end 91.0403 92.0812) (width 0.3048) (layer F.Cu) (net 3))
 (segment (start 91.0403 92.0812) (end 91.0403 112.8043) (width 0.3048) (layer F.Cu) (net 3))
 (segment (start 91.0403 112.8043) (end 94.314 116.078) (width 0.3048) (layer F.Cu) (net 3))
 (segment (start 73.914 127) (end 75.5715 127) (width 0.3048) (layer B.Cu) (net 20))
 (segment (start 75.5715 127) (end 75.5715 131.1891) (width 0.3048) (layer B.Cu) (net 20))
 (segment (start 75.5715 131.1891) (end 81.6337 137.2513) (width 0.3048) (layer B.Cu) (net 20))
 (segment (start 81.6337 137.2513) (end 92.8727 137.2513) (width 0.3048) (layer B.Cu) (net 20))
 (segment (start 92.8727 137.2513) (end 94.234 135.89) (width 0.3048) (layer B.Cu) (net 20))
 (segment (start 94.234 134.5825) (end 83.8014 124.1499) (width 0.3048) (layer F.Cu) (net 20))
 (segment (start 83.8014 124.1499) (end 83.8014 106.6549) (width 0.3048) (layer F.Cu) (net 20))
 (segment (start 83.8014 106.6549) (end 83.1915 106.045) (width 0.3048) (layer F.Cu) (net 20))
 (segment (start 94.234 135.89) (end 94.234 134.5825) (width 0.3048) (layer F.Cu) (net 20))
 (segment (start 81.534 106.045) (end 83.1915 106.045) (width 0.3048) (layer F.Cu) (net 20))
 (segment (start 99.949 89.535) (end 99.949 93.3327) (width 0.3048) (layer F.Cu) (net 17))
 (segment (start 99.949 93.3327) (end 92.329 100.9527) (width 0.3048) (layer F.Cu) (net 17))
 (segment (start 92.329 100.9527) (end 92.329 102.235) (width 0.3048) (layer F.Cu) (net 17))
 (segment (start 81.534 100.965) (end 83.1915 100.965) (width 0.3048) (layer B.Cu) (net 17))
 (segment (start 92.329 102.235) (end 84.4615 102.235) (width 0.3048) (layer B.Cu) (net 17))
 (segment (start 84.4615 102.235) (end 83.1915 100.965) (width 0.3048) (layer B.Cu) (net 17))
 (segment (start 81.534 98.425) (end 79.8765 98.425) (width 0.3048) (layer B.Cu) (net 15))
 (segment (start 58.674 106.045) (end 62.484 102.235) (width 0.3048) (layer B.Cu) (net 15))
 (segment (start 62.484 102.235) (end 76.0665 102.235) (width 0.3048) (layer B.Cu) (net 15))
 (segment (start 76.0665 102.235) (end 79.8765 98.425) (width 0.3048) (layer B.Cu) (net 15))
 (segment (start 92.329 95.885) (end 91.0715 95.885) (width 0.3048) (layer B.Cu) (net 15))
 (segment (start 81.534 98.425) (end 88.5315 98.425) (width 0.3048) (layer B.Cu) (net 15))
 (segment (start 88.5315 98.425) (end 91.0715 95.885) (width 0.3048) (layer B.Cu) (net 15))
 (segment (start 81.534 93.345) (end 79.8765 93.345) (width 0.3048) (layer F.Cu) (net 11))
 (segment (start 78.994 86.995) (end 78.994 92.4625) (width 0.3048) (layer F.Cu) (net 11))
 (segment (start 78.994 92.4625) (end 79.8765 93.345) (width 0.3048) (layer F.Cu) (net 11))
 (segment (start 68.246 157.226) (end 68.199 157.179) (width 0.3048) (layer F.Cu) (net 6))
 (segment (start 68.199 157.179) (end 68.199 149.86) (width 0.3048) (layer F.Cu) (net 6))
 (segment (start 80.184 157.226) (end 80.184 149.86) (width 0.3048) (layer F.Cu) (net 10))
 (segment (start 91.614 157.226) (end 91.694 157.146) (width 0.3048) (layer F.Cu) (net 8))
 (segment (start 91.694 157.146) (end 91.694 150.114) (width 0.3048) (layer F.Cu) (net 8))
 (segment (start 85.979 143.51) (end 84.7215 143.51) (width 0.3048) (layer F.Cu) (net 25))
 (segment (start 81.534 142.8812) (end 84.0927 142.8812) (width 0.3048) (layer F.Cu) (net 25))
 (segment (start 84.0927 142.8812) (end 84.7215 143.51) (width 0.3048) (layer F.Cu) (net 25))
 (segment (start 81.534 142.8812) (end 81.534 142.2525) (width 0.3048) (layer F.Cu) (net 25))
 (segment (start 81.534 143.51) (end 81.534 142.8812) (width 0.3048) (layer F.Cu) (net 25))
 (segment (start 81.534 143.51) (end 80.2765 143.51) (width 0.3048) (layer B.Cu) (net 25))
 (segment (start 80.2765 143.51) (end 79.0109 142.2444) (width 0.3048) (layer B.Cu) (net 25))
 (segment (start 79.0109 142.2444) (end 71.9921 142.2444) (width 0.3048) (layer B.Cu) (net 25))
 (segment (start 71.9921 142.2444) (end 70.7265 143.51) (width 0.3048) (layer B.Cu) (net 25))
 (segment (start 69.469 143.51) (end 70.7265 143.51) (width 0.3048) (layer B.Cu) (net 25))
 (segment (start 58.674 137.795) (end 59.9315 137.795) (width 0.3048) (layer B.Cu) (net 25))
 (segment (start 59.9315 137.795) (end 65.6465 143.51) (width 0.3048) (layer B.Cu) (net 25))
 (segment (start 65.6465 143.51) (end 69.469 143.51) (width 0.3048) (layer B.Cu) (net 25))
 (segment (start 73.914 121.92) (end 75.5715 121.92) (width 0.3048) (layer F.Cu) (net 25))
 (segment (start 75.5715 121.92) (end 78.3079 124.6564) (width 0.3048) (layer F.Cu) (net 25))
 (segment (start 78.3079 124.6564) (end 78.3079 139.0264) (width 0.3048) (layer F.Cu) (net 25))
 (segment (start 78.3079 139.0264) (end 81.534 142.2525) (width 0.3048) (layer F.Cu) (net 25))
 (segment (start 61.849 143.51) (end 65.699 147.36) (width 0.3048) (layer F.Cu) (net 5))
 (segment (start 65.699 147.36) (end 65.699 149.86) (width 0.3048) (layer F.Cu) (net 5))
 (segment (start 73.914 143.51) (end 77.684 147.28) (width 0.3048) (layer B.Cu) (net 9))
 (segment (start 77.684 147.28) (end 77.684 149.86) (width 0.3048) (layer B.Cu) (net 9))
 (segment (start 93.599 143.51) (end 93.599 145.709) (width 0.3048) (layer B.Cu) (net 7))
 (segment (start 93.599 145.709) (end 89.194 150.114) (width 0.3048) (layer B.Cu) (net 7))
 (segment (start 62.5458 131.445) (end 62.5458 134.0468) (width 0.3048) (layer F.Cu) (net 26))
 (segment (start 62.5458 134.0468) (end 66.294 137.795) (width 0.3048) (layer F.Cu) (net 26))
 (segment (start 72.2565 119.38) (end 72.2565 121.7343) (width 0.3048) (layer F.Cu) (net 26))
 (segment (start 72.2565 121.7343) (end 62.5458 131.445) (width 0.3048) (layer F.Cu) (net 26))
 (segment (start 62.5458 131.445) (end 58.674 131.445) (width 0.3048) (layer F.Cu) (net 26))
 (segment (start 73.914 119.38) (end 72.2565 119.38) (width 0.3048) (layer F.Cu) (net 26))
 (segment (start 66.294 131.445) (end 67.5515 131.445) (width 0.3048) (layer F.Cu) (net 27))
 (segment (start 73.914 132.08) (end 68.1865 132.08) (width 0.3048) (layer F.Cu) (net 27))
 (segment (start 68.1865 132.08) (end 67.5515 131.445) (width 0.3048) (layer F.Cu) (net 27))
 (segment (start 66.294 131.445) (end 65.0365 131.445) (width 0.3048) (layer B.Cu) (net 27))
 (segment (start 65.0365 131.445) (end 58.6865 125.095) (width 0.3048) (layer B.Cu) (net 27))
 (segment (start 58.6865 125.095) (end 58.674 125.095) (width 0.3048) (layer B.Cu) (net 27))
 (segment (start 66.294 125.095) (end 66.294 123.8375) (width 0.3048) (layer F.Cu) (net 28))
 (segment (start 66.294 86.995) (end 66.294 88.2525) (width 0.3048) (layer F.Cu) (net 28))
 (segment (start 66.294 88.2525) (end 64.9919 89.5546) (width 0.3048) (layer F.Cu) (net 28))
 (segment (start 64.9919 89.5546) (end 64.9919 110.3065) (width 0.3048) (layer F.Cu) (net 28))
 (segment (start 64.9919 110.3065) (end 66.294 111.6086) (width 0.3048) (layer F.Cu) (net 28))
 (segment (start 66.294 111.6086) (end 66.294 113.0926) (width 0.3048) (layer F.Cu) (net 28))
 (segment (start 66.294 113.0926) (end 65.0018 114.3848) (width 0.3048) (layer F.Cu) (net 28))
 (segment (start 65.0018 114.3848) (end 65.0018 122.5453) (width 0.3048) (layer F.Cu) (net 28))
 (segment (start 65.0018 122.5453) (end 66.294 123.8375) (width 0.3048) (layer F.Cu) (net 28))
 (segment (start 66.294 125.095) (end 66.294 126.3525) (width 0.3048) (layer B.Cu) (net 28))
 (segment (start 73.914 134.62) (end 72.2565 134.62) (width 0.3048) (layer B.Cu) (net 28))
 (segment (start 72.2565 134.62) (end 72.2565 132.315) (width 0.3048) (layer B.Cu) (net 28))
 (segment (start 72.2565 132.315) (end 66.294 126.3525) (width 0.3048) (layer B.Cu) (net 28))
 (segment (start 91.694 130.175) (end 92.964 130.175) (width 0.3048) (layer F.Cu) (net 2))
 (segment (start 92.964 130.175) (end 99.314 123.825) (width 0.3048) (layer F.Cu) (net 2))
 (segment (start 91.694 130.175) (end 90.4365 130.175) (width 0.3048) (layer B.Cu) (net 2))
 (segment (start 81.534 132.08) (end 88.5315 132.08) (width 0.3048) (layer B.Cu) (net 2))
 (segment (start 88.5315 132.08) (end 90.4365 130.175) (width 0.3048) (layer B.Cu) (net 2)))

